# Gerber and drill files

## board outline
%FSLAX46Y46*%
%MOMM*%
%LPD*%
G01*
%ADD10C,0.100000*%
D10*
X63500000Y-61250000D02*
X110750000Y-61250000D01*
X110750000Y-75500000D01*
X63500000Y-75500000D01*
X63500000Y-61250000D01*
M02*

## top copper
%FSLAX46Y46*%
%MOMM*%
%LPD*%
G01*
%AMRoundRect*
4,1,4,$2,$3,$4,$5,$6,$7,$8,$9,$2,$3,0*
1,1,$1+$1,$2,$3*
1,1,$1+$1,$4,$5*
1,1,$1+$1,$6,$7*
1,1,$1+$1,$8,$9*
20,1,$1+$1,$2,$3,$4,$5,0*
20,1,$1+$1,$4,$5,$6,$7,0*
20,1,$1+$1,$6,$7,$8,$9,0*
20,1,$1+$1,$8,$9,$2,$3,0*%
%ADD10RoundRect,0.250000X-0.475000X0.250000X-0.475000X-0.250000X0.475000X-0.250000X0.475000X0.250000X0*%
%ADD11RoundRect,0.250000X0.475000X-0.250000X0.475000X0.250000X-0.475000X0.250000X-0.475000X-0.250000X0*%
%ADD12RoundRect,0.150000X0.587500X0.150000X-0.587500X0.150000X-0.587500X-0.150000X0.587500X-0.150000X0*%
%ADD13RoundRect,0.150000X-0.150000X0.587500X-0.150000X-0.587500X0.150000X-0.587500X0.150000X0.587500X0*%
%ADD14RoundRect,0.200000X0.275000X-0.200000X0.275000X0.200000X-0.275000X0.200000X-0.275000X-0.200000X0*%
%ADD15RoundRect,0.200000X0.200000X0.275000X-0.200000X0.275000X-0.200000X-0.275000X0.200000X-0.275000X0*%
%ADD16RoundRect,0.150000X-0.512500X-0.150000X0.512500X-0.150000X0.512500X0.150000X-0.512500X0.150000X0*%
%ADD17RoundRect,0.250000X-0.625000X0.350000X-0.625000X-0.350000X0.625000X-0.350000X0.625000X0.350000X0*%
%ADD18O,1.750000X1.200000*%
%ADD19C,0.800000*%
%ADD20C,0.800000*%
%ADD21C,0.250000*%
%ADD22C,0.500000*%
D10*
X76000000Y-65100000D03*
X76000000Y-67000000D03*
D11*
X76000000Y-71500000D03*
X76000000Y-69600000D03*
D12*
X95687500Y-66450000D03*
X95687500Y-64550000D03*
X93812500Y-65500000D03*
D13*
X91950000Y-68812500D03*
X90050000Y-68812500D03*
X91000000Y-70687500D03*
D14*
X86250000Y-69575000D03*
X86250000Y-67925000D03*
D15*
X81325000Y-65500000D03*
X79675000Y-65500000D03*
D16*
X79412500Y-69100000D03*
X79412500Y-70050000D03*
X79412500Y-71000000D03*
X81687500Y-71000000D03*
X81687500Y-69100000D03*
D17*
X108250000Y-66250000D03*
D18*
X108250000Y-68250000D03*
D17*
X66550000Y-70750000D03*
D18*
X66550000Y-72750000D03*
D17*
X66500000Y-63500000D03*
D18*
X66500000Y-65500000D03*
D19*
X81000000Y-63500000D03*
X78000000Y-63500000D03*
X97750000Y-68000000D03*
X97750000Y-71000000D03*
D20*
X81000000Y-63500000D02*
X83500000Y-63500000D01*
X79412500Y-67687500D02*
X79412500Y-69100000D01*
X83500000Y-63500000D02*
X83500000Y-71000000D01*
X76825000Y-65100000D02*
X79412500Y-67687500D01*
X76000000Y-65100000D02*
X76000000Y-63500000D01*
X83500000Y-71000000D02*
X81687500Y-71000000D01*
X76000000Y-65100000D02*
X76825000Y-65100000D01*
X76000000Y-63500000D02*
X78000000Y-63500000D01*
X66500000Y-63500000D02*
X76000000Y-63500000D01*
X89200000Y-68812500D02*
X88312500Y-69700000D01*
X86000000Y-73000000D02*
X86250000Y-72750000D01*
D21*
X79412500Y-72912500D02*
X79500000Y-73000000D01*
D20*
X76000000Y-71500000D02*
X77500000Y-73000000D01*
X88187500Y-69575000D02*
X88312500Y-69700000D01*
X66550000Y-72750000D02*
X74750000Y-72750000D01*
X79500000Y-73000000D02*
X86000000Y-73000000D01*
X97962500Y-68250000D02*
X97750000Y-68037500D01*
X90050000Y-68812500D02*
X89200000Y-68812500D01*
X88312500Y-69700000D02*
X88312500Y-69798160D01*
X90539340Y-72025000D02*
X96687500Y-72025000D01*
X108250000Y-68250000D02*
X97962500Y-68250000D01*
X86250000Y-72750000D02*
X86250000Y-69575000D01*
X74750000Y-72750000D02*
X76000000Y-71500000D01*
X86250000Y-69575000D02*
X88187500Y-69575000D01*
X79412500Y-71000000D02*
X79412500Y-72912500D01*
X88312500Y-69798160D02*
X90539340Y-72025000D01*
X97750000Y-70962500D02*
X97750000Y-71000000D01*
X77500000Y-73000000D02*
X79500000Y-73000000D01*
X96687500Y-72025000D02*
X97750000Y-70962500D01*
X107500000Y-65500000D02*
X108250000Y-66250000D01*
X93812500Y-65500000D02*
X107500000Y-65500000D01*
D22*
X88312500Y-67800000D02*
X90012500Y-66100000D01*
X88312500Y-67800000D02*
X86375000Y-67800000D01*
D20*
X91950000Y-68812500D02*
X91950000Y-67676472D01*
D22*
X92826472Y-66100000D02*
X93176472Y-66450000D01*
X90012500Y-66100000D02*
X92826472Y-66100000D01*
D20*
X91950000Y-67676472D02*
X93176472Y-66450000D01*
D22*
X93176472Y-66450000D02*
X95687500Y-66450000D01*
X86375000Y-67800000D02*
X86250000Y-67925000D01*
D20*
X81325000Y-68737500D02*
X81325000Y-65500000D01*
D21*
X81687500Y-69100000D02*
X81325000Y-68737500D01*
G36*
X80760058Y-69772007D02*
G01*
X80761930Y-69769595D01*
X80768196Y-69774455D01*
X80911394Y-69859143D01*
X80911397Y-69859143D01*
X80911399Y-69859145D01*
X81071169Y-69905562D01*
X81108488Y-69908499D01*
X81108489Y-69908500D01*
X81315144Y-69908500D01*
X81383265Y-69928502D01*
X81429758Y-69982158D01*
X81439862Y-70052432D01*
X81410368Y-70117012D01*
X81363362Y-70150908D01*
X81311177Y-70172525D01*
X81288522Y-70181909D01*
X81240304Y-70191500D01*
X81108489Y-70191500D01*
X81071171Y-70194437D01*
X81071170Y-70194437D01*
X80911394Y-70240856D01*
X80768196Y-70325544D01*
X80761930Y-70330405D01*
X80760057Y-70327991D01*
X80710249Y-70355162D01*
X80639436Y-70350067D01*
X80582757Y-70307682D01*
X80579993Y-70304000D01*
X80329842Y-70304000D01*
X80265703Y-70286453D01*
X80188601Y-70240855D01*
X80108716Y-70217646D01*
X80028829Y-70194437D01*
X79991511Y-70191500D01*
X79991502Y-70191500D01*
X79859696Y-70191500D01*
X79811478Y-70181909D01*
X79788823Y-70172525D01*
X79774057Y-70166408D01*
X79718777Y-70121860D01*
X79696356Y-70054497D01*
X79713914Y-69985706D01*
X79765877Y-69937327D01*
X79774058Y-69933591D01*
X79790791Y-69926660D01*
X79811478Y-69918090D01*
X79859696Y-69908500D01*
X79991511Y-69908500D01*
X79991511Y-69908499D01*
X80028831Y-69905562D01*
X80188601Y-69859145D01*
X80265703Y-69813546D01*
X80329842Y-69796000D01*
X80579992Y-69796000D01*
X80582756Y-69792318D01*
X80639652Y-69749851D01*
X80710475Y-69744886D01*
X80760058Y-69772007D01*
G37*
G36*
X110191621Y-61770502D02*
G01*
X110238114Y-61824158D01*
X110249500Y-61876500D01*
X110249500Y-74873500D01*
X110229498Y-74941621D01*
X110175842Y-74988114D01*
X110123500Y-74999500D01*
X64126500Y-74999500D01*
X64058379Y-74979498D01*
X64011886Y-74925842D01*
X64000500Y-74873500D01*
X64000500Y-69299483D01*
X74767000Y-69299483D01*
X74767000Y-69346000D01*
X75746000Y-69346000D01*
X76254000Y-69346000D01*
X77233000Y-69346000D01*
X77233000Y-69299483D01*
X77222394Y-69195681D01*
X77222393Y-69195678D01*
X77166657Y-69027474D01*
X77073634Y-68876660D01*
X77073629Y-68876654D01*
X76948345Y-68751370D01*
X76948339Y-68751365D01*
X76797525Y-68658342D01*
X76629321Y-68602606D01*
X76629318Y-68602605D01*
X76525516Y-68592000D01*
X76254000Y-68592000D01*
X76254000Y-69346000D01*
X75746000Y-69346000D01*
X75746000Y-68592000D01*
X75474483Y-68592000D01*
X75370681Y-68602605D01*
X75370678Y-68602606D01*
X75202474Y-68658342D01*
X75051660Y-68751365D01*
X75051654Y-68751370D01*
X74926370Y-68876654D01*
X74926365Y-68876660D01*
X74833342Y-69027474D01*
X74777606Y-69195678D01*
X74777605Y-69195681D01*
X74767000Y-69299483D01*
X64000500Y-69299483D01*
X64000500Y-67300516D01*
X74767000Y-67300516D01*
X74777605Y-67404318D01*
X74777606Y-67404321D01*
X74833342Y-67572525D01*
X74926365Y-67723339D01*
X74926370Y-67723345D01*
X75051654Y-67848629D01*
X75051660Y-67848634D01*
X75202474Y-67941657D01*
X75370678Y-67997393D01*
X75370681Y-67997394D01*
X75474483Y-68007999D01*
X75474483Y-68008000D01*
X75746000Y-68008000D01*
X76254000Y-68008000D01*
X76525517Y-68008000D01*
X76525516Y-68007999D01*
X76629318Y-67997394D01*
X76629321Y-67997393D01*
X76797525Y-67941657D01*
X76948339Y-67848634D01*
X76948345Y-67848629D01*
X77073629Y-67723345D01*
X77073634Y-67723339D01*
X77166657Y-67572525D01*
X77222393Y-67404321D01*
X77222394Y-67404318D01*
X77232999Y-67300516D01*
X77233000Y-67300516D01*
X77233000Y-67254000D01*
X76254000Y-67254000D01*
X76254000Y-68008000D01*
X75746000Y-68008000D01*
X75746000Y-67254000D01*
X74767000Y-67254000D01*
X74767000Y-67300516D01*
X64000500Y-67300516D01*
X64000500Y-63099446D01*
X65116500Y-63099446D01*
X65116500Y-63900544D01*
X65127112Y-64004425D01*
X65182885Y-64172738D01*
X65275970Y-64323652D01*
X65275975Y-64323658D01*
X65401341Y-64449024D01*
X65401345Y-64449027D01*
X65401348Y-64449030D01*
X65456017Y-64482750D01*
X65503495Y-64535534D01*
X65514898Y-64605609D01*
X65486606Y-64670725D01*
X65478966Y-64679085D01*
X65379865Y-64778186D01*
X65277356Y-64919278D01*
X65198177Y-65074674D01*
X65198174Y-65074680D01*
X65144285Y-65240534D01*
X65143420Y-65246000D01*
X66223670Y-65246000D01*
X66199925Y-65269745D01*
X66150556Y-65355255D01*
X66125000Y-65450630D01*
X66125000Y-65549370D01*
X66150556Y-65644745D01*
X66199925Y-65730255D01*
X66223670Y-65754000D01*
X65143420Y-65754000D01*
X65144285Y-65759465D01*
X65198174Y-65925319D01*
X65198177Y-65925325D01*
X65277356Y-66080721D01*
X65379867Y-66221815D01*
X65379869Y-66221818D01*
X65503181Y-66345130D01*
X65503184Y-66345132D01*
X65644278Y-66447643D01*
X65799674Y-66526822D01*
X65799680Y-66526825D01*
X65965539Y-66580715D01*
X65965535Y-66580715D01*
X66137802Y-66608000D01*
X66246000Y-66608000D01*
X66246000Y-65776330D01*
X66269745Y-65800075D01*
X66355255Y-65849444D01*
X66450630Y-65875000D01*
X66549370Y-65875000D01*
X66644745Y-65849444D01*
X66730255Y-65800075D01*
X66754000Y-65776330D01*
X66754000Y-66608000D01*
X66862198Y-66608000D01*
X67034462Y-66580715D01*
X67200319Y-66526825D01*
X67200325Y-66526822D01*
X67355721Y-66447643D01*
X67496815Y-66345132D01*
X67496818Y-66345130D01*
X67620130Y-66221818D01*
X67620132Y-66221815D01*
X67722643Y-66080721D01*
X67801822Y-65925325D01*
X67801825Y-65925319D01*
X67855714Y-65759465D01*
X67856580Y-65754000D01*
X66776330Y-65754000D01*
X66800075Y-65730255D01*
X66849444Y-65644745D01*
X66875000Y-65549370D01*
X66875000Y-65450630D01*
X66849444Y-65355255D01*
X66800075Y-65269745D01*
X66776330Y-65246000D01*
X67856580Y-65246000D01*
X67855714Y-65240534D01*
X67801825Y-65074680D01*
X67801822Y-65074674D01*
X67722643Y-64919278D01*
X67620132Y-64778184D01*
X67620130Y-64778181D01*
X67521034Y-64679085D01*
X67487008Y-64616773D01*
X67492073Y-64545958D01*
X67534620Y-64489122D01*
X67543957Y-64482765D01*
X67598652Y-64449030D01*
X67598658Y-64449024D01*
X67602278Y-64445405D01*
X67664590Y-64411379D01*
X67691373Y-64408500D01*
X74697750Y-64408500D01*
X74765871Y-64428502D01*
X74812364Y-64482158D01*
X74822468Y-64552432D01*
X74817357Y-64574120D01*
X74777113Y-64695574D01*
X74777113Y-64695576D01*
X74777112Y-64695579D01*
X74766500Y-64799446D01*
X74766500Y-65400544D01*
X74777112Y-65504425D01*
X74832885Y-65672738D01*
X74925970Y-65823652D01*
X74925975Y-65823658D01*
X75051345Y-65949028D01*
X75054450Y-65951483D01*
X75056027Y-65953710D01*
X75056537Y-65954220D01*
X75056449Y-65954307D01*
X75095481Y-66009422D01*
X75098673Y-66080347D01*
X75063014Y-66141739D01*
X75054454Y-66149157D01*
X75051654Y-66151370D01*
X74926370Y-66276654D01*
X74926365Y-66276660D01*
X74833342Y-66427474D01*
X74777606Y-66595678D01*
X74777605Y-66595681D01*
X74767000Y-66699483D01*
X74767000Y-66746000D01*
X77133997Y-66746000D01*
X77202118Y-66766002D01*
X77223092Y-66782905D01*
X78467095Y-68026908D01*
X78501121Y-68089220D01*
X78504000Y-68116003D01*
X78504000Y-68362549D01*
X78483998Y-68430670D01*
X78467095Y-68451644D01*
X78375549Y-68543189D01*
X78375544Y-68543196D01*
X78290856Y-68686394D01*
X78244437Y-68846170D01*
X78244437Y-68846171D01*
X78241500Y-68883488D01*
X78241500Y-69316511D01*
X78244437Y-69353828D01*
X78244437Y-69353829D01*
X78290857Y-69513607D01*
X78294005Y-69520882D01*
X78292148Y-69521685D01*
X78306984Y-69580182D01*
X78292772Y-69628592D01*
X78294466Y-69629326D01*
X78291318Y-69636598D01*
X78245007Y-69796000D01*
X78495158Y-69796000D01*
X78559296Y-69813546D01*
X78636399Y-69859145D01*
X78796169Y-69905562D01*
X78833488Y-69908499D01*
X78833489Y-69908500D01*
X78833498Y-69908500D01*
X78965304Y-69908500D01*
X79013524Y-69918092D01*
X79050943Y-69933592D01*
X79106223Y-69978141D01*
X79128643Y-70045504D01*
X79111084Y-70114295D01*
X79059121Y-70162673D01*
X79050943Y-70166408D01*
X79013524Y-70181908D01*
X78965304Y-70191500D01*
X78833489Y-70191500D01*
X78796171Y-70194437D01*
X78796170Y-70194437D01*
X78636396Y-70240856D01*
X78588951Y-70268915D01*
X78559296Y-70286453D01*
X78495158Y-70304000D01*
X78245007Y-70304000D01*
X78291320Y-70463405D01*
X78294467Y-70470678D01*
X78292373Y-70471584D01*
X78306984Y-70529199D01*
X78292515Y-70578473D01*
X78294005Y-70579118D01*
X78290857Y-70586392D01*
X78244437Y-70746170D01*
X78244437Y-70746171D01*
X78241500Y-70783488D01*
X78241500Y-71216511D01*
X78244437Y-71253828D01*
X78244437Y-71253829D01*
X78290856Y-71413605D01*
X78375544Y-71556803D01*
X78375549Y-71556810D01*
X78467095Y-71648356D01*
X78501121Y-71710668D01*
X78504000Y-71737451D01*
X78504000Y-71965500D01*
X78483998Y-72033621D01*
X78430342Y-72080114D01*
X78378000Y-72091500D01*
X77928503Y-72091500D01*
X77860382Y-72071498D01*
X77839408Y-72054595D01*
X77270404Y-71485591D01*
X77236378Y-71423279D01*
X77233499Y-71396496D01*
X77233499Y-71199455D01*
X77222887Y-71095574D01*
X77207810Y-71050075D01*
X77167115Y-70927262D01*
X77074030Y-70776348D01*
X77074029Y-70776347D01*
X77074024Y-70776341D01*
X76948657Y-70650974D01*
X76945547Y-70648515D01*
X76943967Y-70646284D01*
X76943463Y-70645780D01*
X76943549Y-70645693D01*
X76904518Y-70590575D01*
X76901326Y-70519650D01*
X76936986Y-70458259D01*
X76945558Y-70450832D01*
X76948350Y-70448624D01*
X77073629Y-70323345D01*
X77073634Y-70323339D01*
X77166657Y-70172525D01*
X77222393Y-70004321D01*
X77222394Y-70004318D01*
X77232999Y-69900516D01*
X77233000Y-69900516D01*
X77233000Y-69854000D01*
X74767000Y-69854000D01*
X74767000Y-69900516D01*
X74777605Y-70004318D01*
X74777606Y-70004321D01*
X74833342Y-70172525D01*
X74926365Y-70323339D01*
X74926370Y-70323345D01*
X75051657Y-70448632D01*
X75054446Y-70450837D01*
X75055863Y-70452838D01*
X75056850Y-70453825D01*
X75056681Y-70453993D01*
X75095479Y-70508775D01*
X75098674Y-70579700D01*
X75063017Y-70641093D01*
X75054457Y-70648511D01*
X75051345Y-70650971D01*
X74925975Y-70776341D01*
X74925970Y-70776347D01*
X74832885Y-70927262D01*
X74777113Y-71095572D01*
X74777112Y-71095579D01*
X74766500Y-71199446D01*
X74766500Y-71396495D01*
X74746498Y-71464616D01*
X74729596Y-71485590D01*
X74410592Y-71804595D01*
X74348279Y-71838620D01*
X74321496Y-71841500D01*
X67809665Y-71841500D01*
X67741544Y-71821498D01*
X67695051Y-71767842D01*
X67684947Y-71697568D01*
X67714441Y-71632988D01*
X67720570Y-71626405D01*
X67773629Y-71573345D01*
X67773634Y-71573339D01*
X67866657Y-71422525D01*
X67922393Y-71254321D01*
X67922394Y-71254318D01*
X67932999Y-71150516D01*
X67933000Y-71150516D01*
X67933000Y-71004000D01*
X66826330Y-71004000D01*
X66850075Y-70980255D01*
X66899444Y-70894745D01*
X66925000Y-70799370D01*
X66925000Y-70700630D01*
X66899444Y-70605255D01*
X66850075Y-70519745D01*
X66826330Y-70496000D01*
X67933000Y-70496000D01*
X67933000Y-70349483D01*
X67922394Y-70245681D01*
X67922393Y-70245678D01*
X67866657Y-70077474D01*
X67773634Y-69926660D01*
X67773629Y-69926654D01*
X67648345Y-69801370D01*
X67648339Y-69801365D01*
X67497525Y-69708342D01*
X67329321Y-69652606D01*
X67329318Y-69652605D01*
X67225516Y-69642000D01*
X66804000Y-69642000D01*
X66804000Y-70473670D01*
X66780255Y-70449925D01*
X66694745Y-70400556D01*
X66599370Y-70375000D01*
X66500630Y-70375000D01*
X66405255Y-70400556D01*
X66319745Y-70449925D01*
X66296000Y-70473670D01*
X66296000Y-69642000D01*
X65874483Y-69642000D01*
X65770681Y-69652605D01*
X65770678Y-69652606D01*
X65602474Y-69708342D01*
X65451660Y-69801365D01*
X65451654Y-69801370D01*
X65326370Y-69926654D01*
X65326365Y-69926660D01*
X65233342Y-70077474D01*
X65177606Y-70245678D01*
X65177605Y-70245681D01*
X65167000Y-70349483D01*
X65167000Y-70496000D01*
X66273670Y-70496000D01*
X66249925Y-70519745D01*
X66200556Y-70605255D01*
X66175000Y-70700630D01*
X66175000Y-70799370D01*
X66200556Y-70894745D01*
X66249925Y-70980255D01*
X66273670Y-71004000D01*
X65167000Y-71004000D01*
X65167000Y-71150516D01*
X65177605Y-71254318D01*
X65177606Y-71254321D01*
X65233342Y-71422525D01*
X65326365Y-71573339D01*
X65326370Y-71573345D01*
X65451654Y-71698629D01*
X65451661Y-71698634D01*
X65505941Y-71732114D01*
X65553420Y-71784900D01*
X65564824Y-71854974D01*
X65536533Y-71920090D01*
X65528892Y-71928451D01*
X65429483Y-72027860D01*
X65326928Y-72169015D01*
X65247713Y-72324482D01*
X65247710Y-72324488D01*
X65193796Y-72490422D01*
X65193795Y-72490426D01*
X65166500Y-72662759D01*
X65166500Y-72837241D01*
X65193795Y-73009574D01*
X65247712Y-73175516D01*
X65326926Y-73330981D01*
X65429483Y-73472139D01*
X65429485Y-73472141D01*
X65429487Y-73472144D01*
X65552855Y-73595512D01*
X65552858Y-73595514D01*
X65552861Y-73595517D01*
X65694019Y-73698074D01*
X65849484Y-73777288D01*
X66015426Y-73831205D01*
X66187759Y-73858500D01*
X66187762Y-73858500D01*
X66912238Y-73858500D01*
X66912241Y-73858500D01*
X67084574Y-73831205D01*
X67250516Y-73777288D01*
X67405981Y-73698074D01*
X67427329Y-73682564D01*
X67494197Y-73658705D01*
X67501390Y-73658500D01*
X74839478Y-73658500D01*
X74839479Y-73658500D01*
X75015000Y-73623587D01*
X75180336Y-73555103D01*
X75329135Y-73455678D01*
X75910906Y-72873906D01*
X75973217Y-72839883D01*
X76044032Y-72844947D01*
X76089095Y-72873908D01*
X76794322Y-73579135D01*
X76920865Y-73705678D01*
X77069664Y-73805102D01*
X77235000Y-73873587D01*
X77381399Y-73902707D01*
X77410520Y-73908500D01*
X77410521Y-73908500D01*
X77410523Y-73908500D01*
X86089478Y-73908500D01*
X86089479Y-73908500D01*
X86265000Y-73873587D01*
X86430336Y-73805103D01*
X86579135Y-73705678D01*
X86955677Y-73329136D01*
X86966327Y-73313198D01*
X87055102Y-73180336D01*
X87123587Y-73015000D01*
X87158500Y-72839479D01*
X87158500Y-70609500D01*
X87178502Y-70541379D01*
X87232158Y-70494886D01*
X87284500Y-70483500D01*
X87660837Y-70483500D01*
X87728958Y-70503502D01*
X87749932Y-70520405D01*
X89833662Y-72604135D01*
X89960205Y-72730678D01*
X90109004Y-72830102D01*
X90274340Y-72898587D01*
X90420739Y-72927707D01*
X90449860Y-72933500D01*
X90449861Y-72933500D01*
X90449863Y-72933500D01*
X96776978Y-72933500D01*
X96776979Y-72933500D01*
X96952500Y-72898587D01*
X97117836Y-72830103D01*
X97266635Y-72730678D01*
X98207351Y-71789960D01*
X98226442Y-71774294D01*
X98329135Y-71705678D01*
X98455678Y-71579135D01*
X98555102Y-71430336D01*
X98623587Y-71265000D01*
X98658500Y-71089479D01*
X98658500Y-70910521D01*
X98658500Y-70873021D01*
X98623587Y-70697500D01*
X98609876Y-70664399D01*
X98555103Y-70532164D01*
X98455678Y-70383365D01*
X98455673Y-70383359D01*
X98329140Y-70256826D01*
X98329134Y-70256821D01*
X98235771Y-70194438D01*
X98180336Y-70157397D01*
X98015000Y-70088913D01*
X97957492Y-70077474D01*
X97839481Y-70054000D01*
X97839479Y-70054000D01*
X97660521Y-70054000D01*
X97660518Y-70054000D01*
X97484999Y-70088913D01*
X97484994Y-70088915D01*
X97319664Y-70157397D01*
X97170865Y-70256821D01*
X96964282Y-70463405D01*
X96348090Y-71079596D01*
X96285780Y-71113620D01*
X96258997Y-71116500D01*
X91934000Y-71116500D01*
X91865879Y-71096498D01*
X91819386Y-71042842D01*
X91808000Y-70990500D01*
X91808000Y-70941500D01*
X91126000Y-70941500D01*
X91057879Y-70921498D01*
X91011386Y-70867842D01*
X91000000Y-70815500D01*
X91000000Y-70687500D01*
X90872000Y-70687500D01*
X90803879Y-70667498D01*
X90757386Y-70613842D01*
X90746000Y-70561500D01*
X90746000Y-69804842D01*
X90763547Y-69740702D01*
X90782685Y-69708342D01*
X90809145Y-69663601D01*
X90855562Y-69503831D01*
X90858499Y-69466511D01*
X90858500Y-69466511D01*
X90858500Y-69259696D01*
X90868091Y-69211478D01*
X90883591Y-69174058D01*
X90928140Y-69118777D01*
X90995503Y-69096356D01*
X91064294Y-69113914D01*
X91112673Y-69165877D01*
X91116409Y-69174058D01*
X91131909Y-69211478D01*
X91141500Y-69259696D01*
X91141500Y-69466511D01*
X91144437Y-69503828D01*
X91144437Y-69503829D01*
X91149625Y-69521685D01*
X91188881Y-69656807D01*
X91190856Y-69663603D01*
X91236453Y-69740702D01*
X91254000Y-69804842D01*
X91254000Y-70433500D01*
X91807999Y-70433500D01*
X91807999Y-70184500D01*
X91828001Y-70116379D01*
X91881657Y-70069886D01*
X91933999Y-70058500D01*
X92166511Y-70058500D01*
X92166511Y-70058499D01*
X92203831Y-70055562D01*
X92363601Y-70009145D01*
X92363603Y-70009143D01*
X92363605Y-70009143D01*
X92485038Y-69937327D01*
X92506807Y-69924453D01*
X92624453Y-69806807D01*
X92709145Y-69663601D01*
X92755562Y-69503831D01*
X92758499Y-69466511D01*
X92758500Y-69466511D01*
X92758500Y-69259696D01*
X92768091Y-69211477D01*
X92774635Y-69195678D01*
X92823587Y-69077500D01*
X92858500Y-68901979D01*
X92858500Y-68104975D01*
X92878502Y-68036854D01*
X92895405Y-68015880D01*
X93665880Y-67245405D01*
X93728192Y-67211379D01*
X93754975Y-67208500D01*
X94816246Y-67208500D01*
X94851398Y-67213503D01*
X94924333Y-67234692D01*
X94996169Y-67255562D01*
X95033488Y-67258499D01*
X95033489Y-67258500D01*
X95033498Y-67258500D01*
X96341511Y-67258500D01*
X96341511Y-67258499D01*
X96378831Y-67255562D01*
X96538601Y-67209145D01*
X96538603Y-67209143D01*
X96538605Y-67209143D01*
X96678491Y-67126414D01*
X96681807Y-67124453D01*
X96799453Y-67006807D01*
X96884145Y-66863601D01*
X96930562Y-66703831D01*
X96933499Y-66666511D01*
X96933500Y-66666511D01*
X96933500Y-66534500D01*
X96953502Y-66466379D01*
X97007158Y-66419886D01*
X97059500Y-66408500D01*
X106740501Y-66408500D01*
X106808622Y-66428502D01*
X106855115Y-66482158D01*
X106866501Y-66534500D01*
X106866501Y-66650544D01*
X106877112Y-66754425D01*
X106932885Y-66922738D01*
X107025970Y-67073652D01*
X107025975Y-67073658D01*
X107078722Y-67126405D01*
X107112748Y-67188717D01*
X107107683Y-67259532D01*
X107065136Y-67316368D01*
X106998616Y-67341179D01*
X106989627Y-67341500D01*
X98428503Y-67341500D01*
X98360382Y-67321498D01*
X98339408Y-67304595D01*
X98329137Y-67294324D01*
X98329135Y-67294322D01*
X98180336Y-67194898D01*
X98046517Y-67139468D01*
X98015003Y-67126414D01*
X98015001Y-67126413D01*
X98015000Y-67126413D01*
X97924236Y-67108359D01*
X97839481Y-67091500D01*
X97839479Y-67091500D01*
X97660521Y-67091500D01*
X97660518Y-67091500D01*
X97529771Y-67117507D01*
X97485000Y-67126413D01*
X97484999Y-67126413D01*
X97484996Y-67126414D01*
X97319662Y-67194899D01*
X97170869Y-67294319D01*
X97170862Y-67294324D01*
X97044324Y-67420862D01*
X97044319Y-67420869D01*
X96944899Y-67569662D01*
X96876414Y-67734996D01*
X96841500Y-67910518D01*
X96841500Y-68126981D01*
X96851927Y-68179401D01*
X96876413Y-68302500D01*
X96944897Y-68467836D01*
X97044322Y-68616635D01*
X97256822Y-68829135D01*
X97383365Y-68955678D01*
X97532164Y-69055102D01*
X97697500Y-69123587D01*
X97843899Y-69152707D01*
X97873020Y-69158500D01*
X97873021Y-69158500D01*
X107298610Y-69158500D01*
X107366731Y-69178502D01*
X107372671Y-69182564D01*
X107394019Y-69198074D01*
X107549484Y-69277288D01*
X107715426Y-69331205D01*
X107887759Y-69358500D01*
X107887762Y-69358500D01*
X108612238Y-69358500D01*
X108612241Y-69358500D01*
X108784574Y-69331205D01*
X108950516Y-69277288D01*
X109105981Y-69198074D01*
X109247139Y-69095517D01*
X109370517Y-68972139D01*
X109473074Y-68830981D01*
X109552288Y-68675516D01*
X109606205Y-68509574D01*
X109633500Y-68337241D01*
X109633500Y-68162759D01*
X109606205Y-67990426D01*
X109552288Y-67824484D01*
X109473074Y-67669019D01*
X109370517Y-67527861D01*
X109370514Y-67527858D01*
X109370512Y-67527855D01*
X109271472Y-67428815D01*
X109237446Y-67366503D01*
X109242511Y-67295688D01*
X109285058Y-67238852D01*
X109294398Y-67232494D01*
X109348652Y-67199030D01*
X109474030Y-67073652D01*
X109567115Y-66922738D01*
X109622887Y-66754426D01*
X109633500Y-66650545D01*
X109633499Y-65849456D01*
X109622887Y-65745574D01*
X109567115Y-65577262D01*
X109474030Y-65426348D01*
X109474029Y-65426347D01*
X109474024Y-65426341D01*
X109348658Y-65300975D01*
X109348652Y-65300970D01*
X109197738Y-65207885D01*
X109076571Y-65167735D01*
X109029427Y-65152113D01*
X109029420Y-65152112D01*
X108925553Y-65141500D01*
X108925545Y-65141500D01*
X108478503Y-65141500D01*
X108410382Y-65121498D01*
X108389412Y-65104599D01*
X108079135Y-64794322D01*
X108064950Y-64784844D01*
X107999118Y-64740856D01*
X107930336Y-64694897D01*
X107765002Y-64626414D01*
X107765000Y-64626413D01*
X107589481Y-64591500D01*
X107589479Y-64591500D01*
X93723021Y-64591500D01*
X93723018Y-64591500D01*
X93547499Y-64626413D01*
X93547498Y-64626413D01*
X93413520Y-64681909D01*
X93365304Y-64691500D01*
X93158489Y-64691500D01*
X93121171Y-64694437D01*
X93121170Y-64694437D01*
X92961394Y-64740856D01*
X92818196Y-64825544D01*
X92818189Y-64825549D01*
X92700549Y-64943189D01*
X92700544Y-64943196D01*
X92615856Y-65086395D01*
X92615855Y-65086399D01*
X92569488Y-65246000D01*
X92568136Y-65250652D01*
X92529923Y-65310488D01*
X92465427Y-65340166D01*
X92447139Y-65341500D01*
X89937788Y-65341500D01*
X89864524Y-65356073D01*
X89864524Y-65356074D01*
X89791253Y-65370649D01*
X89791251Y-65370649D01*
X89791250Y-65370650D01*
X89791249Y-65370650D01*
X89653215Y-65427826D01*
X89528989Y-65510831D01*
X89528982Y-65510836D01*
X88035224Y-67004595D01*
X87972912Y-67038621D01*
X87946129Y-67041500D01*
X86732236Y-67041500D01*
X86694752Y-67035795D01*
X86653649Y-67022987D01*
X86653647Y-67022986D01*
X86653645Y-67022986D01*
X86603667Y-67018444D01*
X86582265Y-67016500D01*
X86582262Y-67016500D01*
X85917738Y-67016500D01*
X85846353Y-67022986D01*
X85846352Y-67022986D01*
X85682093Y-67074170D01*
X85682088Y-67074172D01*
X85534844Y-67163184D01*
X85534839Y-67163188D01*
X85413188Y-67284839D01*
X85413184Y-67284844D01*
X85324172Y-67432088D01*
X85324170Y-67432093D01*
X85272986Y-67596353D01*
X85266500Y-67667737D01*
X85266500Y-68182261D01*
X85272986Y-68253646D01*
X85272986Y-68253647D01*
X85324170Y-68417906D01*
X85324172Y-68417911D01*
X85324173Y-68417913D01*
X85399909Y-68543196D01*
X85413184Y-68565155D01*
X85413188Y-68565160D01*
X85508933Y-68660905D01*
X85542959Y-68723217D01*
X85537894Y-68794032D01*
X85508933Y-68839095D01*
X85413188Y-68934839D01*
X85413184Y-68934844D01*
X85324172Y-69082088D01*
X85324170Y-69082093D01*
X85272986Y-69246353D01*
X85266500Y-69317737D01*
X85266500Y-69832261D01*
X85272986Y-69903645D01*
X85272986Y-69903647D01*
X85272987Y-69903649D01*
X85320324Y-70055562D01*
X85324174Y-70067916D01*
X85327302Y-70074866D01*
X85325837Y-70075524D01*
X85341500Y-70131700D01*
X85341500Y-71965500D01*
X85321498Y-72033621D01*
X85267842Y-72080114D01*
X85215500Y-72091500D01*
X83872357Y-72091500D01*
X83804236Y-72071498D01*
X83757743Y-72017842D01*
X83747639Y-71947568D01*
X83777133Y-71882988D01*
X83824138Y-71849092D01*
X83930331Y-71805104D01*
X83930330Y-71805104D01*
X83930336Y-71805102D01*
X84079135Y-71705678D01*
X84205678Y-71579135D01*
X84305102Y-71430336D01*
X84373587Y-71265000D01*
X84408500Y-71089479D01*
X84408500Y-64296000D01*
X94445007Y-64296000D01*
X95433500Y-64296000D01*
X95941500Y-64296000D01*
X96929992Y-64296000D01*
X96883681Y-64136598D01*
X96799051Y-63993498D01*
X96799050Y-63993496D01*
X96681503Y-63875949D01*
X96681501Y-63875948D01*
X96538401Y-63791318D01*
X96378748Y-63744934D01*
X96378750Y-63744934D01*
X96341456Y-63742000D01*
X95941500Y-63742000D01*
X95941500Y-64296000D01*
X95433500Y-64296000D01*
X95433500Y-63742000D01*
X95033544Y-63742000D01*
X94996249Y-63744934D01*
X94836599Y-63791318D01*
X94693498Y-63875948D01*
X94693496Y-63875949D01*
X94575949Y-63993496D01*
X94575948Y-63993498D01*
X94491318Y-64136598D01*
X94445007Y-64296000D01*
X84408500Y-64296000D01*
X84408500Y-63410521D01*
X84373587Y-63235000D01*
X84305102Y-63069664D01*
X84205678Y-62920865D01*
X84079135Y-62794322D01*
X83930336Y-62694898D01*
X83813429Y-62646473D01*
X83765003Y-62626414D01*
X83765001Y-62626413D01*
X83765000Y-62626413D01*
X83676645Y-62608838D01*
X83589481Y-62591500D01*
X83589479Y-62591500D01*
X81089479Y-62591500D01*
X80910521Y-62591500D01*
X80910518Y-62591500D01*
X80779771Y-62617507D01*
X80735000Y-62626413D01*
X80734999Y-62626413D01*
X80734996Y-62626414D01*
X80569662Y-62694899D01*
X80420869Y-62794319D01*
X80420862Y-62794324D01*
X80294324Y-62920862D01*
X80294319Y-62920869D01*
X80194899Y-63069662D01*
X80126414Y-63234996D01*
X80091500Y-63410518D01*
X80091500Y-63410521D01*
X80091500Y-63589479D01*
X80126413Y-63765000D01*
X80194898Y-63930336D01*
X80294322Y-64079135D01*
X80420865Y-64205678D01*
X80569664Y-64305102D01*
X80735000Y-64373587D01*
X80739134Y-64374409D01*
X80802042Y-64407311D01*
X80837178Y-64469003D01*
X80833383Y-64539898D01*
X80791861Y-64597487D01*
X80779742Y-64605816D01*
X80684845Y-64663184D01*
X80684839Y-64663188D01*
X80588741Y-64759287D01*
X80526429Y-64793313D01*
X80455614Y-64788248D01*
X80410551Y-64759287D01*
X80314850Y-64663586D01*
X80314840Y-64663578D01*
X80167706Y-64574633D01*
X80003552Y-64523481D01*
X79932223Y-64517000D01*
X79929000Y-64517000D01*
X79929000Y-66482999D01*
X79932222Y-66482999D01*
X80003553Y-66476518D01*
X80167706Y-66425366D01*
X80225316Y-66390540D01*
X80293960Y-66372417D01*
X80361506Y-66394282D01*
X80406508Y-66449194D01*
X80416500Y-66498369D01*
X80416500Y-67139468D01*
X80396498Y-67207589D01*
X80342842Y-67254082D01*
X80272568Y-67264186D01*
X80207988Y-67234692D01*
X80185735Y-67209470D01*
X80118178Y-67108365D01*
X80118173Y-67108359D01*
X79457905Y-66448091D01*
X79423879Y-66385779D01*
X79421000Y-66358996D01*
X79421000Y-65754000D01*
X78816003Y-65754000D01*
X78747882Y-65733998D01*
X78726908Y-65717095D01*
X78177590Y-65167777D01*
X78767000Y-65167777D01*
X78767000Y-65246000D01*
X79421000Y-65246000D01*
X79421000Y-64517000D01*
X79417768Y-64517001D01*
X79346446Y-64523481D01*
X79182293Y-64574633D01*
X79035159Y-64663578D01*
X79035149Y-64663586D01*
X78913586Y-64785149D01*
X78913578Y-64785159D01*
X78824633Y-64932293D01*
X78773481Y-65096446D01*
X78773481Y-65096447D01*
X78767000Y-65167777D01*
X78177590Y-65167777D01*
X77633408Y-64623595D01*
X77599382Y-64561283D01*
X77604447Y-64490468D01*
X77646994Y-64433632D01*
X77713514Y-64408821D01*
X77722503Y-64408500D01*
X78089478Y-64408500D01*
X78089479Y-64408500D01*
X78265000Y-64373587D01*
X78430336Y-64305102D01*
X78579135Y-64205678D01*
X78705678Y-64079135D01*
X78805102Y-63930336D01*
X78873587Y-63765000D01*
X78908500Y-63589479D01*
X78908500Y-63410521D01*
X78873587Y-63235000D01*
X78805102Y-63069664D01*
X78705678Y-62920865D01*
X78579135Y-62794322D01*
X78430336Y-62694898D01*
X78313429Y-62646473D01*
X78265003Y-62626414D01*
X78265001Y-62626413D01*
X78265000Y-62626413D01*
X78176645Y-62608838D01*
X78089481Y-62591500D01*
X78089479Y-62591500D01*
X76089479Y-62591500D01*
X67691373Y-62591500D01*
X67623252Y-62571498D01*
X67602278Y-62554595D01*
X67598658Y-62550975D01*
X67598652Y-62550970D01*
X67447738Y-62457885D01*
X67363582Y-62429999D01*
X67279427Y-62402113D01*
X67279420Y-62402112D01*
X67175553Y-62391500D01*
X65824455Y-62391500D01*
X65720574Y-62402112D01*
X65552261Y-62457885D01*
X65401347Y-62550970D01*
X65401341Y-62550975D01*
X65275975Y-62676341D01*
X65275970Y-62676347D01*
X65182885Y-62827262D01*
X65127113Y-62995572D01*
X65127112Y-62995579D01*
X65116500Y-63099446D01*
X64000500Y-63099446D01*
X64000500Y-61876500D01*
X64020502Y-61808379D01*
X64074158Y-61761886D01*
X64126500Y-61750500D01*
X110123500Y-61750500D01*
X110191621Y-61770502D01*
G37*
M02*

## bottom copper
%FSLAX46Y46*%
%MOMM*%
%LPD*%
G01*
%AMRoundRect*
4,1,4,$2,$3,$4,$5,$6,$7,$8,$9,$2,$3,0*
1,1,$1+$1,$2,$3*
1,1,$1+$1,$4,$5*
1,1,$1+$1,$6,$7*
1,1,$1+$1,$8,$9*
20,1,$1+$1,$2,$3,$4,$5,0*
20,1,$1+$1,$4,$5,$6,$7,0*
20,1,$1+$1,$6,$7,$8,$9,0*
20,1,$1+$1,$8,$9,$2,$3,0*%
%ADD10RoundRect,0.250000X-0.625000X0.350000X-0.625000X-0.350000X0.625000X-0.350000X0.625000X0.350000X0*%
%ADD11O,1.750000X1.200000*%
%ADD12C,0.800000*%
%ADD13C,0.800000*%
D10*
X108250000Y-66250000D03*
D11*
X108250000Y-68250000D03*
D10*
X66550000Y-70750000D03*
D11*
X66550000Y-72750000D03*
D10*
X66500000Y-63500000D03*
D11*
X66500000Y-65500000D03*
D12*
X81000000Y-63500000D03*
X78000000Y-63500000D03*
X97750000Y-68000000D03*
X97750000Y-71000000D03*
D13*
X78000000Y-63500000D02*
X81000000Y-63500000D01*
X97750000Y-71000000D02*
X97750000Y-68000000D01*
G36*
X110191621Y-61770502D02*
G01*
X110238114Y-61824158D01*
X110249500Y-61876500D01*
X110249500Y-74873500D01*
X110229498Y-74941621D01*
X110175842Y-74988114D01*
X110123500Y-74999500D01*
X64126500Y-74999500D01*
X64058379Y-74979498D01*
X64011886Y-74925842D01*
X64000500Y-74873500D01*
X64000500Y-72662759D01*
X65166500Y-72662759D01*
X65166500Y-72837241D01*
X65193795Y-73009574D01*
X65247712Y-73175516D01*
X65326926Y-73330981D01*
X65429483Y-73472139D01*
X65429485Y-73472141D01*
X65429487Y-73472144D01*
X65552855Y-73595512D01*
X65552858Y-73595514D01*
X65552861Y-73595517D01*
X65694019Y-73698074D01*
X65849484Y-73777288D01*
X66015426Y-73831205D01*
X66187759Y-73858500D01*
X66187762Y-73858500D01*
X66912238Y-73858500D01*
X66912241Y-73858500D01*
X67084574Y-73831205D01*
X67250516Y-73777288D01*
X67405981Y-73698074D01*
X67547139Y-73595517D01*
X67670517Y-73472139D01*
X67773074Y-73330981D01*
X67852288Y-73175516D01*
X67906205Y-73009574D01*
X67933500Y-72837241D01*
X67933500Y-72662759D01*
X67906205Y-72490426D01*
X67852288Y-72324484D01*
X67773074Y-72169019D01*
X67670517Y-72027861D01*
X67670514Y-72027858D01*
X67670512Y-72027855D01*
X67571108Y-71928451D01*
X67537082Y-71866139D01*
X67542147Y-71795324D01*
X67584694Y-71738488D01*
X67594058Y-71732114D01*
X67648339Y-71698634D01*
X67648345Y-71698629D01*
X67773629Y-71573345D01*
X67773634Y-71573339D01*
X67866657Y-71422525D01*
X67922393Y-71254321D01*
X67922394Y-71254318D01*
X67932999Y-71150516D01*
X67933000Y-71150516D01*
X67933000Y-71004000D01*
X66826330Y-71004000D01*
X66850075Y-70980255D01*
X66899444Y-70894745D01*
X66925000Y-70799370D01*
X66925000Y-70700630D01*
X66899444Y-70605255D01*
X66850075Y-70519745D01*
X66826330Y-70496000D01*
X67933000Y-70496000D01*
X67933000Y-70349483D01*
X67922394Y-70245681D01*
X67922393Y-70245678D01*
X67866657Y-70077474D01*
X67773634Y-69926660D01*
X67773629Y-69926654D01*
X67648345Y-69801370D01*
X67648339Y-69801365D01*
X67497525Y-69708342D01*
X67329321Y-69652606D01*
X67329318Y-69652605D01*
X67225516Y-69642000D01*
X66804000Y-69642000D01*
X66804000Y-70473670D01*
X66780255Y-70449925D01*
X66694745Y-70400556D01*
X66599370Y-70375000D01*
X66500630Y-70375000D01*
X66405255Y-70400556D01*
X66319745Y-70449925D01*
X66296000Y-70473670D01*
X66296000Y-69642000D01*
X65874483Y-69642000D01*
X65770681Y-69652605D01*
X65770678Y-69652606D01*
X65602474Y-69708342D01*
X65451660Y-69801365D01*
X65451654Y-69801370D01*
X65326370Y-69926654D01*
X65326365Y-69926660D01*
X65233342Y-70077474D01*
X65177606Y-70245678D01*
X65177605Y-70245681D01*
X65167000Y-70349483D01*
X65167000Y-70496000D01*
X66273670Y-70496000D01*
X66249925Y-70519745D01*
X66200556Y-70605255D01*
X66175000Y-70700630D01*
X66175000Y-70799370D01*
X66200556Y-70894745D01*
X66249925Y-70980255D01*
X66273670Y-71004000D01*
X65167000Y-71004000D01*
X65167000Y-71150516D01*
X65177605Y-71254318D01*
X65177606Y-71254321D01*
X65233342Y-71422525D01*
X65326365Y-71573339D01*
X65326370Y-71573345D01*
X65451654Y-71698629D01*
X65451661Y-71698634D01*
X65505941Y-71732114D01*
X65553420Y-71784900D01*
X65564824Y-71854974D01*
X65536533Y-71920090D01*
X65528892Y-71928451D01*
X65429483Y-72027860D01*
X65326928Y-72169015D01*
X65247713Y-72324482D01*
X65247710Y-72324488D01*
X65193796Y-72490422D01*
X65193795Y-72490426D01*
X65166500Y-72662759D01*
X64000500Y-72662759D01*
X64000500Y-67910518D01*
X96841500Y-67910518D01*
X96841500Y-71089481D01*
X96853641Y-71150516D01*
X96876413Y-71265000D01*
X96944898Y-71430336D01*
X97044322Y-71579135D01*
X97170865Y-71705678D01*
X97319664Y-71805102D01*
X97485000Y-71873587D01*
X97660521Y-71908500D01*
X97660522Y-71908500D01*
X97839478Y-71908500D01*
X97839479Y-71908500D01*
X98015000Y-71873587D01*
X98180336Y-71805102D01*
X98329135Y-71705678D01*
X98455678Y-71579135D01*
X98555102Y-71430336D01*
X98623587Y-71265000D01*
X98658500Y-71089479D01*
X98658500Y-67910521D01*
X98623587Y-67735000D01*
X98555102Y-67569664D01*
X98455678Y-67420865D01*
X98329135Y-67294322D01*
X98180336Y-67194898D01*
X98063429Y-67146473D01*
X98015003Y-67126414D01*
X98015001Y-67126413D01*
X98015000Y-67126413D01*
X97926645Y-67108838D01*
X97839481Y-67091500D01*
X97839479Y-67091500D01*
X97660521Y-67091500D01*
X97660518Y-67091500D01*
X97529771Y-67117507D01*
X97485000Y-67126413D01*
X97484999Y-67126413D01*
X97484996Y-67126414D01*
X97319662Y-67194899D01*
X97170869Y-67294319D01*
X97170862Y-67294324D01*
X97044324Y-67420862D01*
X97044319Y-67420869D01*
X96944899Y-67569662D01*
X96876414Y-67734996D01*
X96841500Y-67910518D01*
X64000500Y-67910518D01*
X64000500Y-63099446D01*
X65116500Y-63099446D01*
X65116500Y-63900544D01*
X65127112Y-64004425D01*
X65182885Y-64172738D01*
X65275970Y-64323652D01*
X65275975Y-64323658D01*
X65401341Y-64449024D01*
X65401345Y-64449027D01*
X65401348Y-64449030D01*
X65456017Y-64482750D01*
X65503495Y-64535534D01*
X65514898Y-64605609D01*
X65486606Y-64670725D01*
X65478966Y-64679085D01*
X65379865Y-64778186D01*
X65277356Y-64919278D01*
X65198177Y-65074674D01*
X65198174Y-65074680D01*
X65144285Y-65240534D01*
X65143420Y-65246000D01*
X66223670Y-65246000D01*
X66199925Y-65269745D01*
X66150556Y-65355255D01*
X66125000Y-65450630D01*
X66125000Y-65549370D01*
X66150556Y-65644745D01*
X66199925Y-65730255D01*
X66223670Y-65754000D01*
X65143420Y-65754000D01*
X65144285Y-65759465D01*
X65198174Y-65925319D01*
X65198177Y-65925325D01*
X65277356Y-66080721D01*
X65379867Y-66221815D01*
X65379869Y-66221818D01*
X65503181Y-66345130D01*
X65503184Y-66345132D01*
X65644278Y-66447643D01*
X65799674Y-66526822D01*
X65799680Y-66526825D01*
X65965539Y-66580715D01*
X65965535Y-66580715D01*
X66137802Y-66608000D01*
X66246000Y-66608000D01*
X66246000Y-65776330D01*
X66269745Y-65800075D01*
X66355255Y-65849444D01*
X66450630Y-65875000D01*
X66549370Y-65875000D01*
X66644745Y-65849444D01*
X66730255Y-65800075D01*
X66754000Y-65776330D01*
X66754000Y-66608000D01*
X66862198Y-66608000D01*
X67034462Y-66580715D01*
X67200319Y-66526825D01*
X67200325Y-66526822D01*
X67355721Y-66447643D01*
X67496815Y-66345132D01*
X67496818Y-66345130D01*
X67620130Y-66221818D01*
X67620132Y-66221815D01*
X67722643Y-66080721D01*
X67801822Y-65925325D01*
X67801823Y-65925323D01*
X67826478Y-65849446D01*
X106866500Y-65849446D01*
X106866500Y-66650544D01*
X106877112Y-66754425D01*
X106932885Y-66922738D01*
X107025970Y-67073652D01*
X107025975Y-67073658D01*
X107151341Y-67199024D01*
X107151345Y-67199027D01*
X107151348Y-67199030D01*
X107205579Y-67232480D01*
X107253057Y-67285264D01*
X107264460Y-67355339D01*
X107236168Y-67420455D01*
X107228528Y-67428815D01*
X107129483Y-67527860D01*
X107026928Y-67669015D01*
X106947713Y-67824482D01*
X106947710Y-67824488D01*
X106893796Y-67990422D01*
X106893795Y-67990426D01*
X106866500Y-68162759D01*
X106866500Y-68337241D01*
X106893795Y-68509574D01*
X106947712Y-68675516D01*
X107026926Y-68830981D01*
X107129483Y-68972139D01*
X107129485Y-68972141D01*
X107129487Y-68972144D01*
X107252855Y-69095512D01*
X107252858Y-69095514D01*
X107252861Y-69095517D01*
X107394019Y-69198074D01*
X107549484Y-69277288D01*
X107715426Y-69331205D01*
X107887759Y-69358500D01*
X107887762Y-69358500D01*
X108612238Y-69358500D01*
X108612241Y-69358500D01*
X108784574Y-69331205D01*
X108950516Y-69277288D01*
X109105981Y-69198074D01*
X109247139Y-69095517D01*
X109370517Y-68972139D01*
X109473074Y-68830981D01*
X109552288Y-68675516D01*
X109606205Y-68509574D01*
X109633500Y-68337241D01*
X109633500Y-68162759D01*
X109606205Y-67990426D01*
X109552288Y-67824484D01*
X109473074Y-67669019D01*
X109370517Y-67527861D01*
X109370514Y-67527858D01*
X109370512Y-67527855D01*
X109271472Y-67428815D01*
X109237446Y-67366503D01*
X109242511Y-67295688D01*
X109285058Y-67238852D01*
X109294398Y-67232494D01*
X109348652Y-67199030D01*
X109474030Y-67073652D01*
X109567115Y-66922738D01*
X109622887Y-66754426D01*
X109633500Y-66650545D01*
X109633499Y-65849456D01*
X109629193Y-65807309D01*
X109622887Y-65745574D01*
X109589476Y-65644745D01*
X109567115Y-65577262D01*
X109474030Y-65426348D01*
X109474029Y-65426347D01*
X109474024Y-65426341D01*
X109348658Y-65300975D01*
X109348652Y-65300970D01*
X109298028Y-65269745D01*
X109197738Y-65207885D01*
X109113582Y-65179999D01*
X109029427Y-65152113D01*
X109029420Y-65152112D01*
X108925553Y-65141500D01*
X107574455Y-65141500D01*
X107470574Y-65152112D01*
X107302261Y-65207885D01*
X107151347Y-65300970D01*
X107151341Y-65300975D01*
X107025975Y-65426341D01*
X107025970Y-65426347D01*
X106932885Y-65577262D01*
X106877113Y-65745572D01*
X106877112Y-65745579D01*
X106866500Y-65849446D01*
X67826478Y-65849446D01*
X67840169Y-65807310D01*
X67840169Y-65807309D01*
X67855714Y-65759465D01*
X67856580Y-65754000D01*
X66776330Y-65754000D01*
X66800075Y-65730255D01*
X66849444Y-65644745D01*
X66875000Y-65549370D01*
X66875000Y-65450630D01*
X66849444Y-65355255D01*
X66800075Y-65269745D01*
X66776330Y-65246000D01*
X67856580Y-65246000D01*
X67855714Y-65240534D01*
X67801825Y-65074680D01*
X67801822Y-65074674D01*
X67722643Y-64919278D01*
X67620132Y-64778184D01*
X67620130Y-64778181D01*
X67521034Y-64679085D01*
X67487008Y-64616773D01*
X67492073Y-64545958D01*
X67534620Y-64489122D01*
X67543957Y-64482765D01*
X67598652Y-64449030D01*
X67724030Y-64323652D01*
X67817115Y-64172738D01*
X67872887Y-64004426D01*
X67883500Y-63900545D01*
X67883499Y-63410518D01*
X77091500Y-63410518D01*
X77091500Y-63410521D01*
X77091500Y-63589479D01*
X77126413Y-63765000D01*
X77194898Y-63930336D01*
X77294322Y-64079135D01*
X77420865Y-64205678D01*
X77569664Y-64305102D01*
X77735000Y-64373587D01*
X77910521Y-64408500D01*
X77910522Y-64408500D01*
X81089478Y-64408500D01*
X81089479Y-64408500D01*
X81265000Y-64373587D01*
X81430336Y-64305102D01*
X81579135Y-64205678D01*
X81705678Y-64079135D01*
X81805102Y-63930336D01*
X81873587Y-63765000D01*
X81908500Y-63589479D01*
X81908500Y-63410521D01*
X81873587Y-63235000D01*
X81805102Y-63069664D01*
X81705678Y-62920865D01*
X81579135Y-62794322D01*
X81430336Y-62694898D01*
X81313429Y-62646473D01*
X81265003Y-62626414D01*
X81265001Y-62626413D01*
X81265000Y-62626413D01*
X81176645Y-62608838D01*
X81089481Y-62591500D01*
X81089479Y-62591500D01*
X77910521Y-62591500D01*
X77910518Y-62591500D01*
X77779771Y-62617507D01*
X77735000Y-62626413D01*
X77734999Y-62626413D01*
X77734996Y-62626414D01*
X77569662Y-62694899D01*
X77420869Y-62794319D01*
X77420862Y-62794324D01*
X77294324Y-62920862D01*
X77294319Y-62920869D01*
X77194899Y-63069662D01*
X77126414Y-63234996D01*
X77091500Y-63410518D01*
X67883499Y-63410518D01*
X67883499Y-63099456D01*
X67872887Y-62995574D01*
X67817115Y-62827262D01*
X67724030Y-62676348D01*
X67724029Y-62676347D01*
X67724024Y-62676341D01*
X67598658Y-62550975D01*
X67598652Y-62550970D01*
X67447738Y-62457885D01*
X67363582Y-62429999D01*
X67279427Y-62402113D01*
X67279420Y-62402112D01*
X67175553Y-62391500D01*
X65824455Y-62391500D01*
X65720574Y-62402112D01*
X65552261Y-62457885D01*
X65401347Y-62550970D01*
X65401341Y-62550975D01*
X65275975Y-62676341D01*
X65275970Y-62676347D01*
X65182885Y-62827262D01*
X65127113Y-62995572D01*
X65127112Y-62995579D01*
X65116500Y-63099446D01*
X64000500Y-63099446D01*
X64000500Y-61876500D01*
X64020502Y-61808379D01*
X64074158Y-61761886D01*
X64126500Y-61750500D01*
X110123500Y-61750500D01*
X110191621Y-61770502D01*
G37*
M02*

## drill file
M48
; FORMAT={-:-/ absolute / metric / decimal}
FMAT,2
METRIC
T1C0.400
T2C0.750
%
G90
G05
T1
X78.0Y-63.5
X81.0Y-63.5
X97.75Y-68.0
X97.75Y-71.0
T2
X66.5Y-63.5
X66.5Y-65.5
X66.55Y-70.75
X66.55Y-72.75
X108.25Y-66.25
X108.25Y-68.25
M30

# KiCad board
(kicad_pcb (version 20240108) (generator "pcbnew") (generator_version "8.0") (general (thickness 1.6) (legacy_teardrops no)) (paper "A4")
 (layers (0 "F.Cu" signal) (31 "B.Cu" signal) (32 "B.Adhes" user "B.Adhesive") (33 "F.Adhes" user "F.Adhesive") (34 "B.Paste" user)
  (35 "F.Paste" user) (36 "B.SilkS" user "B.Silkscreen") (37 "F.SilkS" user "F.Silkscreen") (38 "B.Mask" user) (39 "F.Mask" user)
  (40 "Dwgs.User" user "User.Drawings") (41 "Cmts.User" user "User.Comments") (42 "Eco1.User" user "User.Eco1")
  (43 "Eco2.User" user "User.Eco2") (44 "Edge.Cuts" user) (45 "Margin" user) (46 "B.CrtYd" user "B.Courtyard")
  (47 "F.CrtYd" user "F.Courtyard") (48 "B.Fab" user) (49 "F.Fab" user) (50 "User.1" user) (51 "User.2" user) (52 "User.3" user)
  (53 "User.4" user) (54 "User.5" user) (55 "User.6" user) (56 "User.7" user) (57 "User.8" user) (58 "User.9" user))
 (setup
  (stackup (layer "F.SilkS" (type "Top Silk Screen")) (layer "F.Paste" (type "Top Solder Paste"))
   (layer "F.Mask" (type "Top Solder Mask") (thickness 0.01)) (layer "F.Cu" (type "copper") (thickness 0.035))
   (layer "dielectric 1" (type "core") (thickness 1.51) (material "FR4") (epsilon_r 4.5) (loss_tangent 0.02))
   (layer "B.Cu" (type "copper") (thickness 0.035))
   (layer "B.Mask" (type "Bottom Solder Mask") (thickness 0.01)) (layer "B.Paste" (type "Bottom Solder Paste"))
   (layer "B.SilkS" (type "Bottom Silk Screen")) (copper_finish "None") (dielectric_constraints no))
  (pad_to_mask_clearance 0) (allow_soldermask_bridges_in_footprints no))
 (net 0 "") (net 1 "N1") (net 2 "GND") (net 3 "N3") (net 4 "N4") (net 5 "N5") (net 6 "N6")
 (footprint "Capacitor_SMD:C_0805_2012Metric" (layer "F.Cu") (at 76 66.05 -90)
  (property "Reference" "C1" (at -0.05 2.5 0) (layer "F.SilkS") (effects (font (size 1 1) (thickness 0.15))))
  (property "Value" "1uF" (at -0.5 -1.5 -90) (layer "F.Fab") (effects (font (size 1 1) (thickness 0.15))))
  (pad "1" smd roundrect (at -0.95 0 270) (size 1 1.45) (layers "F.Cu" "F.Paste" "F.Mask") (roundrect_rratio 0.25) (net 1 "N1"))
  (pad "2" smd roundrect (at 0.95 0 270) (size 1 1.45) (layers "F.Cu" "F.Paste" "F.Mask") (roundrect_rratio 0.25) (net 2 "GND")))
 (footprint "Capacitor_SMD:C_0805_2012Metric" (layer "F.Cu") (at 76 70.55 90)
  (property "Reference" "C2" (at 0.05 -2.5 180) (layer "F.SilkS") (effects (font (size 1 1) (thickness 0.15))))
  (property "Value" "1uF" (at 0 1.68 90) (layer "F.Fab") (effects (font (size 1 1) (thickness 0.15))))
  (pad "1" smd roundrect (at -0.95 0 90) (size 1 1.45) (layers "F.Cu" "F.Paste" "F.Mask") (roundrect_rratio 0.25) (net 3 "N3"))
  (pad "2" smd roundrect (at 0.95 0 90) (size 1 1.45) (layers "F.Cu" "F.Paste" "F.Mask") (roundrect_rratio 0.25) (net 2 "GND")))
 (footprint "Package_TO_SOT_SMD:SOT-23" (layer "F.Cu") (at 94.75 65.5 180)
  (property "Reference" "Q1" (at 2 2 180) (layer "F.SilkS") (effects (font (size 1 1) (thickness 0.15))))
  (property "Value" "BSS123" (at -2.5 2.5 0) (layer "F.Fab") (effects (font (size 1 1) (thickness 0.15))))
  (pad "1" smd roundrect (at -0.9375 -0.95 180) (size 1.475 0.6) (layers "F.Cu" "F.Paste" "F.Mask") (roundrect_rratio 0.25) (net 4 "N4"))
  (pad "2" smd roundrect (at -0.9375 0.95 180) (size 1.475 0.6) (layers "F.Cu" "F.Paste" "F.Mask") (roundrect_rratio 0.25) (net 2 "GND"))
  (pad "3" smd roundrect (at 0.9375 0 180) (size 1.475 0.6) (layers "F.Cu" "F.Paste" "F.Mask") (roundrect_rratio 0.25) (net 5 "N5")))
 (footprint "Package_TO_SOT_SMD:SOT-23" (layer "F.Cu") (at 91 69.75 -90)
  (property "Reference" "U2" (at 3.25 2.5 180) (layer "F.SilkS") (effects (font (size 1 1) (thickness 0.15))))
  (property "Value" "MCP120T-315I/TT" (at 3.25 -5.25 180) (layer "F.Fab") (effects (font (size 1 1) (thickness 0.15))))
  (pad "1" smd roundrect (at -0.9375 -0.95 270) (size 1.475 0.6) (layers "F.Cu" "F.Paste" "F.Mask") (roundrect_rratio 0.25) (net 4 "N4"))
  (pad "2" smd roundrect (at -0.9375 0.95 270) (size 1.475 0.6) (layers "F.Cu" "F.Paste" "F.Mask") (roundrect_rratio 0.25) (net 3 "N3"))
  (pad "3" smd roundrect (at 0.9375 0 270) (size 1.475 0.6) (layers "F.Cu" "F.Paste" "F.Mask") (roundrect_rratio 0.25) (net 2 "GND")))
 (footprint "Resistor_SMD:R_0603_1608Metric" (layer "F.Cu") (at 86.25 68.75 90)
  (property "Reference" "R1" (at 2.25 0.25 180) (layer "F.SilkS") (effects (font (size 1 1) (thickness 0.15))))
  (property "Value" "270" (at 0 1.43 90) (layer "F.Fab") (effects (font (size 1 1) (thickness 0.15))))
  (pad "1" smd roundrect (at -0.825 0 90) (size 0.8 0.95) (layers "F.Cu" "F.Paste" "F.Mask") (roundrect_rratio 0.25) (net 3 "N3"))
  (pad "2" smd roundrect (at 0.825 0 90) (size 0.8 0.95) (layers "F.Cu" "F.Paste" "F.Mask") (roundrect_rratio 0.25) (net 4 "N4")))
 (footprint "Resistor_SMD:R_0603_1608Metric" (layer "F.Cu") (at 80.5 65.5 180)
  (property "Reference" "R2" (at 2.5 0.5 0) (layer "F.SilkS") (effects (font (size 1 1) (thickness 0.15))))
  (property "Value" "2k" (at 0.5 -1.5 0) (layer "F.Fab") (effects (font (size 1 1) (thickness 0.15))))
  (pad "1" smd roundrect (at -0.825 0 180) (size 0.8 0.95) (layers "F.Cu" "F.Paste" "F.Mask") (roundrect_rratio 0.25) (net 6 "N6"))
  (pad "2" smd roundrect (at 0.825 0 180) (size 0.8 0.95) (layers "F.Cu" "F.Paste" "F.Mask") (roundrect_rratio 0.25) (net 2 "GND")))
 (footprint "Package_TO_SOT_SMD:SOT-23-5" (layer "F.Cu") (at 80.55 70.05)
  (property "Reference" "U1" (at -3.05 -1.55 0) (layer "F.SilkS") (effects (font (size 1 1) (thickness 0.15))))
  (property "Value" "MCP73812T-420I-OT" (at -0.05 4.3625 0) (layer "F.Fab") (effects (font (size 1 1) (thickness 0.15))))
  (pad "1" smd roundrect (at -1.1375 -0.95) (size 1.325 0.6) (layers "F.Cu" "F.Paste" "F.Mask") (roundrect_rratio 0.25) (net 1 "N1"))
  (pad "2" smd roundrect (at -1.1375 0) (size 1.325 0.6) (layers "F.Cu" "F.Paste" "F.Mask") (roundrect_rratio 0.25) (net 2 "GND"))
  (pad "3" smd roundrect (at -1.1375 0.95) (size 1.325 0.6) (layers "F.Cu" "F.Paste" "F.Mask") (roundrect_rratio 0.25) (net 3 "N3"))
  (pad "4" smd roundrect (at 1.1375 0.95) (size 1.325 0.6) (layers "F.Cu" "F.Paste" "F.Mask") (roundrect_rratio 0.25) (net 1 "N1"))
  (pad "5" smd roundrect (at 1.1375 -0.95) (size 1.325 0.6) (layers "F.Cu" "F.Paste" "F.Mask") (roundrect_rratio 0.25) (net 6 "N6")))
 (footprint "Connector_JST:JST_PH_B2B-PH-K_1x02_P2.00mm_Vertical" (layer "B.Cu") (at 108.25 66.25 -90)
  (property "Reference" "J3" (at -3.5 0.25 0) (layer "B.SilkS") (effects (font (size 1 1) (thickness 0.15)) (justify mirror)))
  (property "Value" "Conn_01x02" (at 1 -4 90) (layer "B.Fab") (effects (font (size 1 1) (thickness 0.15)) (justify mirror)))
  (pad "1" thru_hole roundrect (at 0 0 270) (size 1.2 1.75) (drill 0.75) (layers "*.Cu" "*.Mask") (remove_unused_layers no)
   (roundrect_rratio 0.2083333333) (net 5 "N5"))
  (pad "2" thru_hole oval (at 2 0 270) (size 1.2 1.75) (drill 0.75) (layers "*.Cu" "*.Mask") (remove_unused_layers no) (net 3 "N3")))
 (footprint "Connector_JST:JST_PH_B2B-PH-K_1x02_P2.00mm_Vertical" (layer "B.Cu") (at 66.55 70.75 -90)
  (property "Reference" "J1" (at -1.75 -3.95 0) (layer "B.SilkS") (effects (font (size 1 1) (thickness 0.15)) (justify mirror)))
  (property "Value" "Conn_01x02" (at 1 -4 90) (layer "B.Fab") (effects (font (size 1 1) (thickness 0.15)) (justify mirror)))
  (pad "1" thru_hole roundrect (at 0 0 270) (size 1.2 1.75) (drill 0.75) (layers "*.Cu" "*.Mask") (remove_unused_layers no)
   (roundrect_rratio 0.2083333333) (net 2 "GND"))
  (pad "2" thru_hole oval (at 2 0 270) (size 1.2 1.75) (drill 0.75) (layers "*.Cu" "*.Mask") (remove_unused_layers no) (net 3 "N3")))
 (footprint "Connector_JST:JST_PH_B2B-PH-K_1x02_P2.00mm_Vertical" (layer "B.Cu") (at 66.5 63.5 -90)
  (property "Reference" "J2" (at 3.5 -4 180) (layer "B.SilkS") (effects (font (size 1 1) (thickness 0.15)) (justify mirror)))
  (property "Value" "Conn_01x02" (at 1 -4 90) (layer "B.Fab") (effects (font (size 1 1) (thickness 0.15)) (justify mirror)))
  (pad "1" thru_hole roundrect (at 0 0 270) (size 1.2 1.75) (drill 0.75) (layers "*.Cu" "*.Mask") (remove_unused_layers no)
   (roundrect_rratio 0.2083333333) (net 1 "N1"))
  (pad "2" thru_hole oval (at 2 0 270) (size 1.2 1.75) (drill 0.75) (layers "*.Cu" "*.Mask") (remove_unused_layers no) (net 2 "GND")))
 (gr_rect (start 63.5 61.25) (end 110.75 75.5) (stroke (width 0.1) (type solid)) (fill none) (layer "Edge.Cuts"))
 (segment (start 81 63.5) (end 83.5 63.5) (width 0.8) (layer "F.Cu") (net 1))
 (segment (start 79.4125 67.6875) (end 79.4125 69.1) (width 0.8) (layer "F.Cu") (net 1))
 (segment (start 83.5 63.5) (end 83.5 71) (width 0.8) (layer "F.Cu") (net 1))
 (segment (start 76.825 65.1) (end 79.4125 67.6875) (width 0.8) (layer "F.Cu") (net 1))
 (segment (start 76 65.1) (end 76 63.5) (width 0.8) (layer "F.Cu") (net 1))
 (segment (start 83.5 71) (end 81.6875 71) (width 0.8) (layer "F.Cu") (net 1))
 (segment (start 76 65.1) (end 76.825 65.1) (width 0.8) (layer "F.Cu") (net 1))
 (segment (start 76 63.5) (end 78 63.5) (width 0.8) (layer "F.Cu") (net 1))
 (segment (start 66.5 63.5) (end 76 63.5) (width 0.8) (layer "F.Cu") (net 1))
 (via (at 81 63.5) (size 0.8) (drill 0.4) (layers "F.Cu" "B.Cu") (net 1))
 (via (at 78 63.5) (size 0.8) (drill 0.4) (layers "F.Cu" "B.Cu") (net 1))
 (segment (start 78 63.5) (end 81 63.5) (width 0.8) (layer "B.Cu") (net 1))
 (segment (start 89.2 68.8125) (end 88.3125 69.7) (width 0.8) (layer "F.Cu") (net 3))
 (segment (start 86 73) (end 86.25 72.75) (width 0.8) (layer "F.Cu") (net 3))
 (segment (start 79.4125 72.9125) (end 79.5 73) (width 0.25) (layer "F.Cu") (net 3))
 (segment (start 76 71.5) (end 77.5 73) (width 0.8) (layer "F.Cu") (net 3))
 (segment (start 88.1875 69.575) (end 88.3125 69.7) (width 0.8) (layer "F.Cu") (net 3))
 (segment (start 66.55 72.75) (end 74.75 72.75) (width 0.8) (layer "F.Cu") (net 3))
 (segment (start 79.5 73) (end 86 73) (width 0.8) (layer "F.Cu") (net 3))
 (segment (start 97.9625 68.25) (end 97.75 68.0375) (width 0.8) (layer "F.Cu") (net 3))
 (segment (start 90.05 68.8125) (end 89.2 68.8125) (width 0.8) (layer "F.Cu") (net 3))
 (segment (start 88.3125 69.7) (end 88.3125 69.79816) (width 0.8) (layer "F.Cu") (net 3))
 (segment (start 90.53934 72.025) (end 96.6875 72.025) (width 0.8) (layer "F.Cu") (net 3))
 (segment (start 108.25 68.25) (end 97.9625 68.25) (width 0.8) (layer "F.Cu") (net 3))
 (segment (start 86.25 72.75) (end 86.25 69.575) (width 0.8) (layer "F.Cu") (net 3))
 (segment (start 74.75 72.75) (end 76 71.5) (width 0.8) (layer "F.Cu") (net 3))
 (segment (start 86.25 69.575) (end 88.1875 69.575) (width 0.8) (layer "F.Cu") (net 3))
 (segment (start 79.4125 71) (end 79.4125 72.9125) (width 0.8) (layer "F.Cu") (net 3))
 (segment (start 88.3125 69.79816) (end 90.53934 72.025) (width 0.8) (layer "F.Cu") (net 3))
 (segment (start 97.75 70.9625) (end 97.75 71) (width 0.8) (layer "F.Cu") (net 3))
 (segment (start 77.5 73) (end 79.5 73) (width 0.8) (layer "F.Cu") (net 3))
 (segment (start 96.6875 72.025) (end 97.75 70.9625) (width 0.8) (layer "F.Cu") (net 3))
 (via (at 97.75 68) (size 0.8) (drill 0.4) (layers "F.Cu" "B.Cu") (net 3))
 (via (at 97.75 71) (size 0.8) (drill 0.4) (layers "F.Cu" "B.Cu") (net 3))
 (segment (start 97.75 71) (end 97.75 68) (width 0.8) (layer "B.Cu") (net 3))
 (segment (start 107.5 65.5) (end 108.25 66.25) (width 0.8) (layer "F.Cu") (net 5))
 (segment (start 93.8125 65.5) (end 107.5 65.5) (width 0.8) (layer "F.Cu") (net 5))
 (segment (start 88.3125 67.8) (end 90.0125 66.1) (width 0.5) (layer "F.Cu") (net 4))
 (segment (start 88.3125 67.8) (end 86.375 67.8) (width 0.5) (layer "F.Cu") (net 4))
 (segment (start 91.95 68.8125) (end 91.95 67.676472) (width 0.8) (layer "F.Cu") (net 4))
 (segment (start 92.826472 66.1) (end 93.176472 66.45) (width 0.5) (layer "F.Cu") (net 4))
 (segment (start 90.0125 66.1) (end 92.826472 66.1) (width 0.5) (layer "F.Cu") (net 4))
 (segment (start 91.95 67.676472) (end 93.176472 66.45) (width 0.8) (layer "F.Cu") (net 4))
 (segment (start 93.176472 66.45) (end 95.6875 66.45) (width 0.5) (layer "F.Cu") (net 4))
 (segment (start 86.375 67.8) (end 86.25 67.925) (width 0.5) (layer "F.Cu") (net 4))
 (segment (start 81.325 68.7375) (end 81.325 65.5) (width 0.8) (layer "F.Cu") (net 6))
 (segment (start 81.6875 69.1) (end 81.325 68.7375) (width 0.25) (layer "F.Cu") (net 6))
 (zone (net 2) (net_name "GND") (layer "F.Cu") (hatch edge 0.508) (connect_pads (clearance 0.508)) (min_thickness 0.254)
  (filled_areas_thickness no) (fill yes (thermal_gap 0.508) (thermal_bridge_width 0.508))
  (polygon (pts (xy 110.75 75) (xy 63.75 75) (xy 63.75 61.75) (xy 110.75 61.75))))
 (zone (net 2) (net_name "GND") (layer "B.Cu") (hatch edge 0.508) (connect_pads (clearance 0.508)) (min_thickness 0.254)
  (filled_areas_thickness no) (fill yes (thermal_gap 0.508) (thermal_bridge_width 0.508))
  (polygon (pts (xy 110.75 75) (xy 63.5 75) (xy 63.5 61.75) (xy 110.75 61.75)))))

